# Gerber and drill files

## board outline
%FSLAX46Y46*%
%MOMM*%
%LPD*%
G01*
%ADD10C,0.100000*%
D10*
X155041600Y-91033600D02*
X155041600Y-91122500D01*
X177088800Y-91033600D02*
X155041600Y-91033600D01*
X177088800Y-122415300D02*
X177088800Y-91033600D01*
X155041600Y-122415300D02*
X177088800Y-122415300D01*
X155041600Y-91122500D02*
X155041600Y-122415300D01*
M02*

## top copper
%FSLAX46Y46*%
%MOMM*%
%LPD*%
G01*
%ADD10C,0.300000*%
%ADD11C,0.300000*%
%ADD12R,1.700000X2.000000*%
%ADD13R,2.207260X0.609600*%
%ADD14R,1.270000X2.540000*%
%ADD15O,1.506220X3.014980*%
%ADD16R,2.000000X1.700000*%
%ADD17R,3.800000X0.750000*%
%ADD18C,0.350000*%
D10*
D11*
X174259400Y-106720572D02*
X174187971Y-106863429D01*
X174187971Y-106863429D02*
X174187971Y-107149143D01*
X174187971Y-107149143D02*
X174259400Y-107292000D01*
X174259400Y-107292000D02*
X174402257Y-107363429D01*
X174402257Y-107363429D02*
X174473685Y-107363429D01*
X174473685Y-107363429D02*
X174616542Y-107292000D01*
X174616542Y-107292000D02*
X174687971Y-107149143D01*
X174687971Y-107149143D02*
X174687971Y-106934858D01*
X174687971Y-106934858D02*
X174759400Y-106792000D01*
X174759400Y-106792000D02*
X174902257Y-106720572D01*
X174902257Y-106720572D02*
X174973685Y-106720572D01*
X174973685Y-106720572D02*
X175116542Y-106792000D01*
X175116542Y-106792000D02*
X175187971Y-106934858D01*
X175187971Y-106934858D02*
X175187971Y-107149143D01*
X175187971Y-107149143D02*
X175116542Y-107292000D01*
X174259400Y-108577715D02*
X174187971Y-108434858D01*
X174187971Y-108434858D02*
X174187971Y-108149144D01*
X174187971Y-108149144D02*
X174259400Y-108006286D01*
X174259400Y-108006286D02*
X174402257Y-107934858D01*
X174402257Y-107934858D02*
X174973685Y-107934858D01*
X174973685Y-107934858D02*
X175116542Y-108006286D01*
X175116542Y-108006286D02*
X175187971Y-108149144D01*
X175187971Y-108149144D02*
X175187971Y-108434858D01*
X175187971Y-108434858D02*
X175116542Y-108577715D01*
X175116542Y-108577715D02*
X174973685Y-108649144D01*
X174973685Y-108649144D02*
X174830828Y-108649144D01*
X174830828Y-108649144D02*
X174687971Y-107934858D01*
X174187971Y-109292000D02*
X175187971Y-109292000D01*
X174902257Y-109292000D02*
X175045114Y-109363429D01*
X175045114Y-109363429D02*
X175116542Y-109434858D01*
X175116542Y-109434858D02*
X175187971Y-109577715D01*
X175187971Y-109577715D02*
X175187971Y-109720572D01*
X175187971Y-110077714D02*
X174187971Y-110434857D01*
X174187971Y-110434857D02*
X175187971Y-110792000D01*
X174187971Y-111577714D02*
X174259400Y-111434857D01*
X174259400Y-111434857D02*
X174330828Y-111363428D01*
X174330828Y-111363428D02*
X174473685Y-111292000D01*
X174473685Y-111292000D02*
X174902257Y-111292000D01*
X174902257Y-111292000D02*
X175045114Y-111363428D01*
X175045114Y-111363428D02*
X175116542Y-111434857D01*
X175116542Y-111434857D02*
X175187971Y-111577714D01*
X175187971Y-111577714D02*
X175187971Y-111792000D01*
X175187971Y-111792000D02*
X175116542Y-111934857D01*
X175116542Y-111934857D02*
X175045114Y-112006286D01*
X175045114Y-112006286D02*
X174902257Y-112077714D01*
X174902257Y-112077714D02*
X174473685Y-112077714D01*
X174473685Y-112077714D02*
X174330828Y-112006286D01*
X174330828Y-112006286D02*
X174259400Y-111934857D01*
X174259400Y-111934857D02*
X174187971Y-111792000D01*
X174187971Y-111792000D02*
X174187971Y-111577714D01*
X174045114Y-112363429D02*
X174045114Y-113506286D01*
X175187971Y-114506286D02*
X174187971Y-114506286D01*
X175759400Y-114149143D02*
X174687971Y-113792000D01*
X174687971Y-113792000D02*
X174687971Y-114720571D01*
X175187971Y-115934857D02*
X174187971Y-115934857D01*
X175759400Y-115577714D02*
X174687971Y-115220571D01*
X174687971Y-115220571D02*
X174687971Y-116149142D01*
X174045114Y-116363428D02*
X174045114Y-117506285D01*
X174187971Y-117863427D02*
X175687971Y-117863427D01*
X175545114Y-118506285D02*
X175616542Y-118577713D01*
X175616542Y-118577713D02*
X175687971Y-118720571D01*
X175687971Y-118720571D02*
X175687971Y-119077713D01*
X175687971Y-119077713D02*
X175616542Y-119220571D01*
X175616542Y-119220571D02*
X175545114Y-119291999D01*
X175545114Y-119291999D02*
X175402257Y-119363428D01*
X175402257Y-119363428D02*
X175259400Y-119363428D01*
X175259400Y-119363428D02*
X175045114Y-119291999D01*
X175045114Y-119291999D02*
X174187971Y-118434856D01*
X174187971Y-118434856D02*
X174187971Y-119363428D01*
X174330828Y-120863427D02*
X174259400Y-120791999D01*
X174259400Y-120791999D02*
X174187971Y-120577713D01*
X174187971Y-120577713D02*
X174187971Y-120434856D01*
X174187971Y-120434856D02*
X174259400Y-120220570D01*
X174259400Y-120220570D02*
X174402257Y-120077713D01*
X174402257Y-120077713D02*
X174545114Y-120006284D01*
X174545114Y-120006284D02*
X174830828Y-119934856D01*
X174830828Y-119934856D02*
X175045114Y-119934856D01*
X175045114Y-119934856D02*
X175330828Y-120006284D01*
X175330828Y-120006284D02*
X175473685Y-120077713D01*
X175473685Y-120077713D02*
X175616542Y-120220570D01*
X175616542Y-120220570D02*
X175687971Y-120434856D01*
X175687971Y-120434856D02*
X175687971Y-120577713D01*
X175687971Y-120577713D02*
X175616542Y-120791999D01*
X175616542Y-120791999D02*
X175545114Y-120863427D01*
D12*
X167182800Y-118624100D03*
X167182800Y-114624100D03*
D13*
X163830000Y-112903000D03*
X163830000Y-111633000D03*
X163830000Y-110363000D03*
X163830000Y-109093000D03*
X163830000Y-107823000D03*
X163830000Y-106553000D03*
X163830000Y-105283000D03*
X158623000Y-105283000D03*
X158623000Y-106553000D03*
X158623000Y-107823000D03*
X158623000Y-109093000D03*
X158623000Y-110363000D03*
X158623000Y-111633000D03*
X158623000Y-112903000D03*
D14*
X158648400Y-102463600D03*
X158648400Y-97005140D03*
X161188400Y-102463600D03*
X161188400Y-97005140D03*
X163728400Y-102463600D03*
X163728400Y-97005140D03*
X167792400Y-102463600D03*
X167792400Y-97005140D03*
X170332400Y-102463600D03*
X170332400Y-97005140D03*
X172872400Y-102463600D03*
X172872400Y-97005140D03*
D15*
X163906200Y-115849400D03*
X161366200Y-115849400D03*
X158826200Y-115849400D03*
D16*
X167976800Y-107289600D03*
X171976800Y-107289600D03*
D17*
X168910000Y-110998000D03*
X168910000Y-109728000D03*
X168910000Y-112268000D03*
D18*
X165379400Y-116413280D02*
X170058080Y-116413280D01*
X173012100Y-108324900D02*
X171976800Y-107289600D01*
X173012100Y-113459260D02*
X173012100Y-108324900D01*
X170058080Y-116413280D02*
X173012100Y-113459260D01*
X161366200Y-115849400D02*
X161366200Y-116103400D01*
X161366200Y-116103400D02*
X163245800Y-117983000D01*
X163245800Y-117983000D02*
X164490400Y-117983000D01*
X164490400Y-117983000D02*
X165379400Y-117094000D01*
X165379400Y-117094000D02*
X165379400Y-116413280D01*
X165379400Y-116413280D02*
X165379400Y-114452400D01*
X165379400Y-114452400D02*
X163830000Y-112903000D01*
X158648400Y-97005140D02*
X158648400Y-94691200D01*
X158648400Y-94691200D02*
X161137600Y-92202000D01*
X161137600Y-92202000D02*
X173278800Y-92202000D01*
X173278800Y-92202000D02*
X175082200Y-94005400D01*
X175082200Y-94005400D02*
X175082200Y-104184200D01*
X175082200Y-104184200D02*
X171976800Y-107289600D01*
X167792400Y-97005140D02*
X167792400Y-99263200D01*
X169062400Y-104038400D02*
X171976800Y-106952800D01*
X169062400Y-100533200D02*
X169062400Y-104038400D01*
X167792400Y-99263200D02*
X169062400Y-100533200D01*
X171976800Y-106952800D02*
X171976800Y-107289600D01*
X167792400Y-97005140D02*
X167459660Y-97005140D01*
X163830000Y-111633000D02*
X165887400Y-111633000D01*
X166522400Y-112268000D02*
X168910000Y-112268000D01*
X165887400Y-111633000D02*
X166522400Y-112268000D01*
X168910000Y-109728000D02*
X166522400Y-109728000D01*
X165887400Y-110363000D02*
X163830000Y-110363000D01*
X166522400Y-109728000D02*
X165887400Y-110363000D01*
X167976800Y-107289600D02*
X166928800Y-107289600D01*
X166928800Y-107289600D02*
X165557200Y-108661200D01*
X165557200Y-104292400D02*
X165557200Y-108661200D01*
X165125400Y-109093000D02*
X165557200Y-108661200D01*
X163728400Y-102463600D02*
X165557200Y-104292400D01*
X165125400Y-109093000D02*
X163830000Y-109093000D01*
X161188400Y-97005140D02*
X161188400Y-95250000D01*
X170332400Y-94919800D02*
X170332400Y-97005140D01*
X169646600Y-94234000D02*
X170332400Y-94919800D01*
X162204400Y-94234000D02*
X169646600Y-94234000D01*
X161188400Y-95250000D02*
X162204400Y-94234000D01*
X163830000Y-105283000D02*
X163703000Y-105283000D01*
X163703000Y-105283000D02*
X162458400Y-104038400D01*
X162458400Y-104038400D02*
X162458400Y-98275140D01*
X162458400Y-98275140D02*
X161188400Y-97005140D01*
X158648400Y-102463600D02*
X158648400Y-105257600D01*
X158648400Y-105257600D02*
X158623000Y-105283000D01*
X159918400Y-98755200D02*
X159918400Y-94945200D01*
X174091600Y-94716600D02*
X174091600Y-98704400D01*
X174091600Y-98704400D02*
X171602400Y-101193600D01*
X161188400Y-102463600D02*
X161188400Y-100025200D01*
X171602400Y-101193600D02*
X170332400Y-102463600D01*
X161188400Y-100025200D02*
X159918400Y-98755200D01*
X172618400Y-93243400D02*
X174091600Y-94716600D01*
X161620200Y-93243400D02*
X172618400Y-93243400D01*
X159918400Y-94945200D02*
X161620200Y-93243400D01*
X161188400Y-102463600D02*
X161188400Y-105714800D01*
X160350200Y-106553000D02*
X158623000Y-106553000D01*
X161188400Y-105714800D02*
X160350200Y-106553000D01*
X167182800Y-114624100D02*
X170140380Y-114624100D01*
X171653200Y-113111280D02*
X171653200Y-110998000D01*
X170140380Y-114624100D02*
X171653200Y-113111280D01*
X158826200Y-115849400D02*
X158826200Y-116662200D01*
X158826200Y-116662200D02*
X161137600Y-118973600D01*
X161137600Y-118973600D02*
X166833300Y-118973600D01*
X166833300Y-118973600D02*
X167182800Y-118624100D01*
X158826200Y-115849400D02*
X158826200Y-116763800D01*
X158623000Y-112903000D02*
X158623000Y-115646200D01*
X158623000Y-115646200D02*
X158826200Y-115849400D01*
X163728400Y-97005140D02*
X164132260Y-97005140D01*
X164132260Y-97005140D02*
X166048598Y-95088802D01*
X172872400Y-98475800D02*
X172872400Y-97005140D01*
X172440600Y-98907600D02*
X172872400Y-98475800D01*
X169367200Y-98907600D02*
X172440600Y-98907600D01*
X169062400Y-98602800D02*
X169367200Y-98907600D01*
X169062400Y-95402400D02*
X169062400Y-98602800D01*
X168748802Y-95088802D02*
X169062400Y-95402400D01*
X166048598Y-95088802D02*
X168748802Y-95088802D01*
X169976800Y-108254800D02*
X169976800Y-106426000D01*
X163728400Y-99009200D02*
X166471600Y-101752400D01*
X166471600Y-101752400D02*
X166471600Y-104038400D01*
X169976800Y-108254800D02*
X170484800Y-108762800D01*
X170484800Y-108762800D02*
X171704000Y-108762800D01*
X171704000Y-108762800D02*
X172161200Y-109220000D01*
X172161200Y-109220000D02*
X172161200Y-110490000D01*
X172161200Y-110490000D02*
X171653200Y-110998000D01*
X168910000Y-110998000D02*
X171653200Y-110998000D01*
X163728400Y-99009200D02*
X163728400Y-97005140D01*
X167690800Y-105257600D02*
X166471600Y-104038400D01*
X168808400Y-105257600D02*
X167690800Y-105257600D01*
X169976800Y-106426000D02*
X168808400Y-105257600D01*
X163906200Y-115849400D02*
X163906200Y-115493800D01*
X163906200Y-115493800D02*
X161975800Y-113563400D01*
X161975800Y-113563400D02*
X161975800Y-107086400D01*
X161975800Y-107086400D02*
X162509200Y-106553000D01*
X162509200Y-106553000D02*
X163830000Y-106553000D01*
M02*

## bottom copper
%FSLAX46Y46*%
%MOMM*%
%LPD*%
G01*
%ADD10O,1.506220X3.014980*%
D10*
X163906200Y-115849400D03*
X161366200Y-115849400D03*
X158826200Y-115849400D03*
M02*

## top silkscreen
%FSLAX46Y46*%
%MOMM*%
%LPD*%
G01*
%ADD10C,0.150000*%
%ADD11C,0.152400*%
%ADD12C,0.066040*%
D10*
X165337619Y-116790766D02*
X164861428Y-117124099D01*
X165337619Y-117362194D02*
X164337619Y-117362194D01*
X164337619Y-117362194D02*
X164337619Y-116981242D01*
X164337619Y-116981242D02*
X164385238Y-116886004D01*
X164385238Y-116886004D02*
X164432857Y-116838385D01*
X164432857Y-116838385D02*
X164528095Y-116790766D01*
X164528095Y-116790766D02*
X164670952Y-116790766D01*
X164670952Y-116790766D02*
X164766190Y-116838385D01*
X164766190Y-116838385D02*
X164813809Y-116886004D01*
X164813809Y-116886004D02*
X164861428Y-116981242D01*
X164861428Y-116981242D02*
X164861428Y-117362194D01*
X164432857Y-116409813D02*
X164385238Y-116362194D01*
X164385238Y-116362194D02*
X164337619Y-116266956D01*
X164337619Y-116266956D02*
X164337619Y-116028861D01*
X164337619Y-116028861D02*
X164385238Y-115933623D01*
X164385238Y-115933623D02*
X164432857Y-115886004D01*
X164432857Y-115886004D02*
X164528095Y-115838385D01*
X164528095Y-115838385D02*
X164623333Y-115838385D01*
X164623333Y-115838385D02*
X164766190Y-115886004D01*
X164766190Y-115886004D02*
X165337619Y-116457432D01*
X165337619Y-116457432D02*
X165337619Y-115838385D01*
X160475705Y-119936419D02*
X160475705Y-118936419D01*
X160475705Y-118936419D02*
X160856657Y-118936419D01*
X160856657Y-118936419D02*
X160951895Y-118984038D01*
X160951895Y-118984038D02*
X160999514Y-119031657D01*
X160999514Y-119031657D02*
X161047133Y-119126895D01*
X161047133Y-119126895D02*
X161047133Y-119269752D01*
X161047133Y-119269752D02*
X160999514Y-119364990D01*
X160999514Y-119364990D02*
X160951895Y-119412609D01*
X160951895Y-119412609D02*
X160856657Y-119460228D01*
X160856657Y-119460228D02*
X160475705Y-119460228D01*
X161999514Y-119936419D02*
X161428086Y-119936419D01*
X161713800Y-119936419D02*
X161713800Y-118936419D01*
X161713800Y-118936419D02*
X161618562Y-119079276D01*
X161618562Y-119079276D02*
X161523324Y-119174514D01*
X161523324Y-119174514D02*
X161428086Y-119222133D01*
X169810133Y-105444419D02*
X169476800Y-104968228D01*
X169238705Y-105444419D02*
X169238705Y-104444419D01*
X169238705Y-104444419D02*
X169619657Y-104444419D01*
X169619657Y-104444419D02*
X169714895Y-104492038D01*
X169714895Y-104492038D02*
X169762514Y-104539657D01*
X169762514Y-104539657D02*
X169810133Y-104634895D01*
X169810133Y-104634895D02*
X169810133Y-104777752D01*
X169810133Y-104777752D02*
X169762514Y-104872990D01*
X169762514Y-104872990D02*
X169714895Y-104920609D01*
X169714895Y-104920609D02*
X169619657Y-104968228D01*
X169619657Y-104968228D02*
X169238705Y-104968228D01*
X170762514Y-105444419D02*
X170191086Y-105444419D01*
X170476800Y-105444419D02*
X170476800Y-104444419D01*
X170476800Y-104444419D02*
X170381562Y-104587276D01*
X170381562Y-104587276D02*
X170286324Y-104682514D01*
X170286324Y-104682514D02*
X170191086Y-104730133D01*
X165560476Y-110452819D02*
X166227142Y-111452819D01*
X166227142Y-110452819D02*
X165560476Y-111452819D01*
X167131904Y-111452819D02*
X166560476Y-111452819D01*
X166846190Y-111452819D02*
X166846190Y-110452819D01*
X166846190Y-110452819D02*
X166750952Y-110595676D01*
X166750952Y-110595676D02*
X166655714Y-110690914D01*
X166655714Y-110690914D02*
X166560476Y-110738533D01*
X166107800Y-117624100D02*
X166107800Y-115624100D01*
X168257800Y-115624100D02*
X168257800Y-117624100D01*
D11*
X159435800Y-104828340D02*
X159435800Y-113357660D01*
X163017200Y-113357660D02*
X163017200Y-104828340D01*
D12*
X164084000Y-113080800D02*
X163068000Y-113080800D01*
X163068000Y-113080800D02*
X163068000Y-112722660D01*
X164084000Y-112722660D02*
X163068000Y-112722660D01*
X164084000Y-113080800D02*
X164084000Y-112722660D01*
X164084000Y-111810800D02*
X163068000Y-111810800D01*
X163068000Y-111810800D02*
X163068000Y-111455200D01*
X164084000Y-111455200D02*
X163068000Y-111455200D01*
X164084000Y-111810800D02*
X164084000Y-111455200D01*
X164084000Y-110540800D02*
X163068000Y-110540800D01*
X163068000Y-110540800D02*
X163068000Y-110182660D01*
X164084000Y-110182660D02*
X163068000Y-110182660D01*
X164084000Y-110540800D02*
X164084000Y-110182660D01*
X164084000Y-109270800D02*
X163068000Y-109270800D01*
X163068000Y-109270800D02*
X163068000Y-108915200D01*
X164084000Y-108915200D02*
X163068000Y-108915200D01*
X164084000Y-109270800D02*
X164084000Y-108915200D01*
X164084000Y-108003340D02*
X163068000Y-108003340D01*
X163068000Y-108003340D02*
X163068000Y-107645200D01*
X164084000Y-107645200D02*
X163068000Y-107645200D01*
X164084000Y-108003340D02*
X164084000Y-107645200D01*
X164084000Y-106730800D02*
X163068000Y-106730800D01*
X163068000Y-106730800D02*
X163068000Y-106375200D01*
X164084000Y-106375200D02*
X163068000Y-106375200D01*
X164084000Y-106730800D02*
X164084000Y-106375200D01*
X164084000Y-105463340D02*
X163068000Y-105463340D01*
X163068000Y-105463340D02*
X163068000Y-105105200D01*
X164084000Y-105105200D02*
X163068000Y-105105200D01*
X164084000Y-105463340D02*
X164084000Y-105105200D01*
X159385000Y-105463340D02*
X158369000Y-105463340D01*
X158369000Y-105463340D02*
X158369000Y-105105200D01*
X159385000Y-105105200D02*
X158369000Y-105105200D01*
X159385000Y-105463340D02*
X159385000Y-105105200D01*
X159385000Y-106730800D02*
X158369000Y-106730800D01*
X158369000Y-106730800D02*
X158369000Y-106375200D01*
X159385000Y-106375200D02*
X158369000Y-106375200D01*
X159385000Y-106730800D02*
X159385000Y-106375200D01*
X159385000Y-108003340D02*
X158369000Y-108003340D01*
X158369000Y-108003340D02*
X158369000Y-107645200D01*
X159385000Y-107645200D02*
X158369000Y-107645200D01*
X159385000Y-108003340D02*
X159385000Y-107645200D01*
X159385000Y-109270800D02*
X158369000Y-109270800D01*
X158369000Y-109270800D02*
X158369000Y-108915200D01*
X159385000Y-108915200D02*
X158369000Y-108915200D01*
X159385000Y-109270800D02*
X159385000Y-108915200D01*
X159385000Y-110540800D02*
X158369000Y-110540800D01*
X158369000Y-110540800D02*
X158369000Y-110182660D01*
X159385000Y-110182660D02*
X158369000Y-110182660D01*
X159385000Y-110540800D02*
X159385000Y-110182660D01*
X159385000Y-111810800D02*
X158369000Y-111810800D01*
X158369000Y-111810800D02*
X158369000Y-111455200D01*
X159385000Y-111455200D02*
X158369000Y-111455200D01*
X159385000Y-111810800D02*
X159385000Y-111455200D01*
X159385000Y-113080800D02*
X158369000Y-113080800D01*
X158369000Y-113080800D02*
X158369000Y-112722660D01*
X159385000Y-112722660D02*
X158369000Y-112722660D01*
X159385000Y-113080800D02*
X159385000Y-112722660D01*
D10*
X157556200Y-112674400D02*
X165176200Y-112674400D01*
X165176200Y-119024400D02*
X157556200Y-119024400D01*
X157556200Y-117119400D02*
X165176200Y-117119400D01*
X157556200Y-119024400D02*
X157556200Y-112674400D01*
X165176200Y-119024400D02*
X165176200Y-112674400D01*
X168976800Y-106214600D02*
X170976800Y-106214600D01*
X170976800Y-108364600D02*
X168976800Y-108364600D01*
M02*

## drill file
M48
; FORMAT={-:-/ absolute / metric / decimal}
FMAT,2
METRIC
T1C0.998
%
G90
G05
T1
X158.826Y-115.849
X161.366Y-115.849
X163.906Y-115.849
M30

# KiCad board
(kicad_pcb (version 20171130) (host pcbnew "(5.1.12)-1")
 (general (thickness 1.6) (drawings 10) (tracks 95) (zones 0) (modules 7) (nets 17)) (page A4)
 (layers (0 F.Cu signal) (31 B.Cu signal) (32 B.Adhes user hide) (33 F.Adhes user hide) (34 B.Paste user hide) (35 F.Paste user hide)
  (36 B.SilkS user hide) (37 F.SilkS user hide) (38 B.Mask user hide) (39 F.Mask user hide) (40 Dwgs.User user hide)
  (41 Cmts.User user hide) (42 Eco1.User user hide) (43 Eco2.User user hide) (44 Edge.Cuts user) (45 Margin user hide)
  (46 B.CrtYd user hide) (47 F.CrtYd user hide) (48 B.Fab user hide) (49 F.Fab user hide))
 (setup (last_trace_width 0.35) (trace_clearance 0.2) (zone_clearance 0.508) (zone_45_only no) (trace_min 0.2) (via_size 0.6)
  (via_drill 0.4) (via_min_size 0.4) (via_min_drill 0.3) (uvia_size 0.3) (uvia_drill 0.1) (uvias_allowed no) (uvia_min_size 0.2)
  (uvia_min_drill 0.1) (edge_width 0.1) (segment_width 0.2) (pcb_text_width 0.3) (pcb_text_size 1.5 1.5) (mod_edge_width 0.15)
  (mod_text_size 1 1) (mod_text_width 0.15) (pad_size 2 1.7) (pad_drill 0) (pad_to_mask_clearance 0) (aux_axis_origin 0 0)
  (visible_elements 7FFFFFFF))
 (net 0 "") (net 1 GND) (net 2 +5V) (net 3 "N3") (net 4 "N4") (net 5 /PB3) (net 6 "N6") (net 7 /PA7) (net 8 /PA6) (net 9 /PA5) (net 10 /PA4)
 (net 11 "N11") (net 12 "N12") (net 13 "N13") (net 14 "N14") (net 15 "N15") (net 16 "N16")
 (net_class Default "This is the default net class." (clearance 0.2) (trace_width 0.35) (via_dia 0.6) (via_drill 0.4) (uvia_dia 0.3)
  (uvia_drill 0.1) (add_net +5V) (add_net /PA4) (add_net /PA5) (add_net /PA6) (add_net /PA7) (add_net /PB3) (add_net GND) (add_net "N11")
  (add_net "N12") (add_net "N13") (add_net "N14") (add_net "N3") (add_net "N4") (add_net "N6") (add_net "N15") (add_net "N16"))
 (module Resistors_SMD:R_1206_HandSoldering (layer F.Cu) (at 167.1828 116.6241 90)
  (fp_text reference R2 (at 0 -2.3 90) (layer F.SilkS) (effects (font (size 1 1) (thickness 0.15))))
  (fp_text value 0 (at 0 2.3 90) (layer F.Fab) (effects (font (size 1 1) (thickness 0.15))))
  (fp_line (start -1 -1.075) (end 1 -1.075) (layer F.SilkS) (width 0.15))
  (fp_line (start 1 1.075) (end -1 1.075) (layer F.SilkS) (width 0.15))
  (pad 2 smd rect (at -2 0 90) (size 2 1.7) (layers F.Cu F.Paste F.Mask) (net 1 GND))
  (pad 1 smd rect (at 2 0 90) (size 2 1.7) (layers F.Cu F.Paste F.Mask) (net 1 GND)))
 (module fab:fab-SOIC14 (layer F.Cu) (at 161.2265 109.093 90)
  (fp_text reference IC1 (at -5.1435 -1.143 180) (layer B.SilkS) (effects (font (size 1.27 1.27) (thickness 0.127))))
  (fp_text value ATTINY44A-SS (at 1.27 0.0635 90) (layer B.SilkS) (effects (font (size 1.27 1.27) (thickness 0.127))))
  (fp_line (start 4.26466 -1.7907) (end -4.26466 -1.7907) (layer F.SilkS) (width 0.1524))
  (fp_line (start -4.26466 1.7907) (end 4.26466 1.7907) (layer F.SilkS) (width 0.1524))
  (fp_line (start -3.9878 2.8575) (end -3.9878 1.8415) (layer F.SilkS) (width 0.06604))
  (fp_line (start -3.9878 1.8415) (end -3.62966 1.8415) (layer F.SilkS) (width 0.06604))
  (fp_line (start -3.62966 2.8575) (end -3.62966 1.8415) (layer F.SilkS) (width 0.06604))
  (fp_line (start -3.9878 2.8575) (end -3.62966 2.8575) (layer F.SilkS) (width 0.06604))
  (fp_line (start -2.7178 2.8575) (end -2.7178 1.8415) (layer F.SilkS) (width 0.06604))
  (fp_line (start -2.7178 1.8415) (end -2.3622 1.8415) (layer F.SilkS) (width 0.06604))
  (fp_line (start -2.3622 2.8575) (end -2.3622 1.8415) (layer F.SilkS) (width 0.06604))
  (fp_line (start -2.7178 2.8575) (end -2.3622 2.8575) (layer F.SilkS) (width 0.06604))
  (fp_line (start -1.4478 2.8575) (end -1.4478 1.8415) (layer F.SilkS) (width 0.06604))
  (fp_line (start -1.4478 1.8415) (end -1.08966 1.8415) (layer F.SilkS) (width 0.06604))
  (fp_line (start -1.08966 2.8575) (end -1.08966 1.8415) (layer F.SilkS) (width 0.06604))
  (fp_line (start -1.4478 2.8575) (end -1.08966 2.8575) (layer F.SilkS) (width 0.06604))
  (fp_line (start -0.1778 2.8575) (end -0.1778 1.8415) (layer F.SilkS) (width 0.06604))
  (fp_line (start -0.1778 1.8415) (end 0.1778 1.8415) (layer F.SilkS) (width 0.06604))
  (fp_line (start 0.1778 2.8575) (end 0.1778 1.8415) (layer F.SilkS) (width 0.06604))
  (fp_line (start -0.1778 2.8575) (end 0.1778 2.8575) (layer F.SilkS) (width 0.06604))
  (fp_line (start 1.08966 2.8575) (end 1.08966 1.8415) (layer F.SilkS) (width 0.06604))
  (fp_line (start 1.08966 1.8415) (end 1.4478 1.8415) (layer F.SilkS) (width 0.06604))
  (fp_line (start 1.4478 2.8575) (end 1.4478 1.8415) (layer F.SilkS) (width 0.06604))
  (fp_line (start 1.08966 2.8575) (end 1.4478 2.8575) (layer F.SilkS) (width 0.06604))
  (fp_line (start 2.3622 2.8575) (end 2.3622 1.8415) (layer F.SilkS) (width 0.06604))
  (fp_line (start 2.3622 1.8415) (end 2.7178 1.8415) (layer F.SilkS) (width 0.06604))
  (fp_line (start 2.7178 2.8575) (end 2.7178 1.8415) (layer F.SilkS) (width 0.06604))
  (fp_line (start 2.3622 2.8575) (end 2.7178 2.8575) (layer F.SilkS) (width 0.06604))
  (fp_line (start 3.62966 2.8575) (end 3.62966 1.8415) (layer F.SilkS) (width 0.06604))
  (fp_line (start 3.62966 1.8415) (end 3.9878 1.8415) (layer F.SilkS) (width 0.06604))
  (fp_line (start 3.9878 2.8575) (end 3.9878 1.8415) (layer F.SilkS) (width 0.06604))
  (fp_line (start 3.62966 2.8575) (end 3.9878 2.8575) (layer F.SilkS) (width 0.06604))
  (fp_line (start 3.62966 -1.8415) (end 3.62966 -2.8575) (layer F.SilkS) (width 0.06604))
  (fp_line (start 3.62966 -2.8575) (end 3.9878 -2.8575) (layer F.SilkS) (width 0.06604))
  (fp_line (start 3.9878 -1.8415) (end 3.9878 -2.8575) (layer F.SilkS) (width 0.06604))
  (fp_line (start 3.62966 -1.8415) (end 3.9878 -1.8415) (layer F.SilkS) (width 0.06604))
  (fp_line (start 2.3622 -1.8415) (end 2.3622 -2.8575) (layer F.SilkS) (width 0.06604))
  (fp_line (start 2.3622 -2.8575) (end 2.7178 -2.8575) (layer F.SilkS) (width 0.06604))
  (fp_line (start 2.7178 -1.8415) (end 2.7178 -2.8575) (layer F.SilkS) (width 0.06604))
  (fp_line (start 2.3622 -1.8415) (end 2.7178 -1.8415) (layer F.SilkS) (width 0.06604))
  (fp_line (start 1.08966 -1.8415) (end 1.08966 -2.8575) (layer F.SilkS) (width 0.06604))
  (fp_line (start 1.08966 -2.8575) (end 1.4478 -2.8575) (layer F.SilkS) (width 0.06604))
  (fp_line (start 1.4478 -1.8415) (end 1.4478 -2.8575) (layer F.SilkS) (width 0.06604))
  (fp_line (start 1.08966 -1.8415) (end 1.4478 -1.8415) (layer F.SilkS) (width 0.06604))
  (fp_line (start -0.1778 -1.8415) (end -0.1778 -2.8575) (layer F.SilkS) (width 0.06604))
  (fp_line (start -0.1778 -2.8575) (end 0.1778 -2.8575) (layer F.SilkS) (width 0.06604))
  (fp_line (start 0.1778 -1.8415) (end 0.1778 -2.8575) (layer F.SilkS) (width 0.06604))
  (fp_line (start -0.1778 -1.8415) (end 0.1778 -1.8415) (layer F.SilkS) (width 0.06604))
  (fp_line (start -1.4478 -1.8415) (end -1.4478 -2.8575) (layer F.SilkS) (width 0.06604))
  (fp_line (start -1.4478 -2.8575) (end -1.08966 -2.8575) (layer F.SilkS) (width 0.06604))
  (fp_line (start -1.08966 -1.8415) (end -1.08966 -2.8575) (layer F.SilkS) (width 0.06604))
  (fp_line (start -1.4478 -1.8415) (end -1.08966 -1.8415) (layer F.SilkS) (width 0.06604))
  (fp_line (start -2.7178 -1.8415) (end -2.7178 -2.8575) (layer F.SilkS) (width 0.06604))
  (fp_line (start -2.7178 -2.8575) (end -2.3622 -2.8575) (layer F.SilkS) (width 0.06604))
  (fp_line (start -2.3622 -1.8415) (end -2.3622 -2.8575) (layer F.SilkS) (width 0.06604))
  (fp_line (start -2.7178 -1.8415) (end -2.3622 -1.8415) (layer F.SilkS) (width 0.06604))
  (fp_line (start -3.9878 -1.8415) (end -3.9878 -2.8575) (layer F.SilkS) (width 0.06604))
  (fp_line (start -3.9878 -2.8575) (end -3.62966 -2.8575) (layer F.SilkS) (width 0.06604))
  (fp_line (start -3.62966 -1.8415) (end -3.62966 -2.8575) (layer F.SilkS) (width 0.06604))
  (fp_line (start -3.9878 -1.8415) (end -3.62966 -1.8415) (layer F.SilkS) (width 0.06604))
  (pad 1 smd rect (at -3.81 2.6035 90) (size 0.6096 2.20726) (layers F.Cu F.Paste F.Mask) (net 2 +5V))
  (pad 2 smd rect (at -2.54 2.6035 90) (size 0.6096 2.20726) (layers F.Cu F.Paste F.Mask) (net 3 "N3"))
  (pad 3 smd rect (at -1.27 2.6035 90) (size 0.6096 2.20726) (layers F.Cu F.Paste F.Mask) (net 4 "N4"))
  (pad 4 smd rect (at 0 2.6035 90) (size 0.6096 2.20726) (layers F.Cu F.Paste F.Mask) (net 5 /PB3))
  (pad 5 smd rect (at 1.27 2.6035 90) (size 0.6096 2.20726) (layers F.Cu F.Paste F.Mask) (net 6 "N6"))
  (pad 6 smd rect (at 2.54 2.6035 90) (size 0.6096 2.20726) (layers F.Cu F.Paste F.Mask) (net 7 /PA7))
  (pad 7 smd rect (at 3.81 2.6035 90) (size 0.6096 2.20726) (layers F.Cu F.Paste F.Mask) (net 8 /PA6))
  (pad 8 smd rect (at 3.81 -2.6035 90) (size 0.6096 2.20726) (layers F.Cu F.Paste F.Mask) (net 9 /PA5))
  (pad 9 smd rect (at 2.54 -2.6035 90) (size 0.6096 2.20726) (layers F.Cu F.Paste F.Mask) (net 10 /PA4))
  (pad 10 smd rect (at 1.27 -2.6035 90) (size 0.6096 2.20726) (layers F.Cu F.Paste F.Mask) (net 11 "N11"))
  (pad 11 smd rect (at 0 -2.6035 90) (size 0.6096 2.20726) (layers F.Cu F.Paste F.Mask) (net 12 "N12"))
  (pad 12 smd rect (at -1.27 -2.6035 90) (size 0.6096 2.20726) (layers F.Cu F.Paste F.Mask) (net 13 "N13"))
  (pad 13 smd rect (at -2.54 -2.6035 90) (size 0.6096 2.20726) (layers F.Cu F.Paste F.Mask) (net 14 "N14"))
  (pad 14 smd rect (at -3.81 -2.6035 90) (size 0.6096 2.20726) (layers F.Cu F.Paste F.Mask) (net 1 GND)))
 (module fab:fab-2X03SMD (layer F.Cu) (at 161.1884 99.9236 90)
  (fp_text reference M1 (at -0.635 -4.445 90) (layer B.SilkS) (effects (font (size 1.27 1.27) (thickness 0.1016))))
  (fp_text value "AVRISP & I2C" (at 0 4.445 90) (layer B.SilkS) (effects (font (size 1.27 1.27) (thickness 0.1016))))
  (pad 1 smd rect (at -2.54 -2.54 90) (size 2.54 1.27) (layers F.Cu F.Paste F.Mask) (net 9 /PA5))
  (pad 2 smd rect (at 2.91846 -2.54 90) (size 2.54 1.27) (layers F.Cu F.Paste F.Mask) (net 2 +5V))
  (pad 3 smd rect (at -2.54 0 90) (size 2.54 1.27) (layers F.Cu F.Paste F.Mask) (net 10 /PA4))
  (pad 4 smd rect (at 2.91846 0 90) (size 2.54 1.27) (layers F.Cu F.Paste F.Mask) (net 8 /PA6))
  (pad 5 smd rect (at -2.54 2.54 90) (size 2.54 1.27) (layers F.Cu F.Paste F.Mask) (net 5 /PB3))
  (pad 6 smd rect (at 2.91846 2.54 90) (size 2.54 1.27) (layers F.Cu F.Paste F.Mask) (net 1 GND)))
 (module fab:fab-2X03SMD (layer F.Cu) (at 170.3324 99.9236 90)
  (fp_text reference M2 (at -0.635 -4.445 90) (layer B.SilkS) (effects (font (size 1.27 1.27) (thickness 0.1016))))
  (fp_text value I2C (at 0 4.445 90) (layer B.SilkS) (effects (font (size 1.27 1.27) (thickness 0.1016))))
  (pad 1 smd rect (at -2.54 -2.54 90) (size 2.54 1.27) (layers F.Cu F.Paste F.Mask) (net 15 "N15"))
  (pad 2 smd rect (at 2.91846 -2.54 90) (size 2.54 1.27) (layers F.Cu F.Paste F.Mask) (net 2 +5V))
  (pad 3 smd rect (at -2.54 0 90) (size 2.54 1.27) (layers F.Cu F.Paste F.Mask) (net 10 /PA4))
  (pad 4 smd rect (at 2.91846 0 90) (size 2.54 1.27) (layers F.Cu F.Paste F.Mask) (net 8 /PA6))
  (pad 5 smd rect (at -2.54 2.54 90) (size 2.54 1.27) (layers F.Cu F.Paste F.Mask) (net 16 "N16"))
  (pad 6 smd rect (at 2.91846 2.54 90) (size 2.54 1.27) (layers F.Cu F.Paste F.Mask) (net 1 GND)))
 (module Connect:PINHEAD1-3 (layer F.Cu) (at 161.3662 115.8494 180)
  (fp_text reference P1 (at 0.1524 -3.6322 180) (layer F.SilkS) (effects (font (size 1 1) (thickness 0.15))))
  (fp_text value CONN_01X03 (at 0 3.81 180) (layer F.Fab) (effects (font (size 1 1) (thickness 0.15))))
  (fp_line (start 3.81 3.175) (end -3.81 3.175) (layer F.SilkS) (width 0.15))
  (fp_line (start -3.81 -3.175) (end 3.81 -3.175) (layer F.SilkS) (width 0.15))
  (fp_line (start 3.81 -1.27) (end -3.81 -1.27) (layer F.SilkS) (width 0.15))
  (fp_line (start 3.81 -3.175) (end 3.81 3.175) (layer F.SilkS) (width 0.15))
  (fp_line (start -3.81 -3.175) (end -3.81 3.175) (layer F.SilkS) (width 0.15))
  (pad 1 thru_hole oval (at -2.54 0 180) (size 1.50622 3.01498) (drill 0.99822) (layers *.Cu *.Mask) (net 7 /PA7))
  (pad 2 thru_hole oval (at 0 0 180) (size 1.50622 3.01498) (drill 0.99822) (layers *.Cu *.Mask) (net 2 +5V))
  (pad 3 thru_hole oval (at 2.54 0 180) (size 1.50622 3.01498) (drill 0.99822) (layers *.Cu *.Mask) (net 1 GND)))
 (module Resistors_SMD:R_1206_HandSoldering (layer F.Cu) (at 169.9768 107.2896)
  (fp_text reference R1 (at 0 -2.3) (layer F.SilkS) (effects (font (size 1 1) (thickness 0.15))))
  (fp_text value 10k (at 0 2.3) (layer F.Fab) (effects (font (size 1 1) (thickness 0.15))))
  (fp_line (start -1 -1.075) (end 1 -1.075) (layer F.SilkS) (width 0.15))
  (fp_line (start 1 1.075) (end -1 1.075) (layer F.SilkS) (width 0.15))
  (pad 1 smd rect (at -2 0) (size 2 1.7) (layers F.Cu F.Paste F.Mask) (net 5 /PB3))
  (pad 2 smd rect (at 2 0) (size 2 1.7) (layers F.Cu F.Paste F.Mask) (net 2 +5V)))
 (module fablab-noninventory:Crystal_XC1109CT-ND (layer F.Cu) (at 168.91 110.998 90)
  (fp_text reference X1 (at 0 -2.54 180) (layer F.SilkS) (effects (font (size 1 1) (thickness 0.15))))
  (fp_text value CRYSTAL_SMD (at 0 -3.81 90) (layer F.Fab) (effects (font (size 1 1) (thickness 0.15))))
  (pad 2 smd rect (at 0 0 90) (size 0.75 3.8) (layers F.Cu F.Paste F.Mask) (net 1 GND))
  (pad 1 smd rect (at 1.27 0 90) (size 0.75 3.8) (layers F.Cu F.Paste F.Mask) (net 4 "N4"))
  (pad 3 smd rect (at -1.27 0 90) (size 0.75 3.8) (layers F.Cu F.Paste F.Mask) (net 3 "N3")))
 (gr_line (start 155.0416 91.0336) (end 155.0416 91.1225) (angle 90) (layer Edge.Cuts) (width 0.1))
 (gr_line (start 177.0888 91.0336) (end 155.0416 91.0336) (angle 90) (layer Edge.Cuts) (width 0.1))
 (gr_line (start 177.0888 122.4153) (end 177.0888 91.0336) (angle 90) (layer Edge.Cuts) (width 0.1))
 (gr_line (start 155.0416 122.4153) (end 177.0888 122.4153) (angle 90) (layer Edge.Cuts) (width 0.1))
 (gr_line (start 155.0416 91.1225) (end 155.0416 122.4153) (angle 90) (layer Edge.Cuts) (width 0.1))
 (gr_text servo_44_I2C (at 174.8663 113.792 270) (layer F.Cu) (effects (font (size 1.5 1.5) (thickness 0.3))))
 (segment (start 165.3794 116.41328) (end 170.05808 116.41328) (width 0.35) (layer F.Cu) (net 2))
 (segment (start 173.0121 108.3249) (end 171.9768 107.2896) (width 0.35) (layer F.Cu) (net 2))
 (segment (start 173.0121 113.45926) (end 173.0121 108.3249) (width 0.35) (layer F.Cu) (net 2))
 (segment (start 170.05808 116.41328) (end 173.0121 113.45926) (width 0.35) (layer F.Cu) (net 2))
 (segment (start 161.3662 115.8494) (end 161.3662 116.1034) (width 0.35) (layer F.Cu) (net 2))
 (segment (start 161.3662 116.1034) (end 163.2458 117.983) (width 0.35) (layer F.Cu) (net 2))
 (segment (start 163.2458 117.983) (end 164.4904 117.983) (width 0.35) (layer F.Cu) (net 2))
 (segment (start 164.4904 117.983) (end 165.3794 117.094) (width 0.35) (layer F.Cu) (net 2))
 (segment (start 165.3794 117.094) (end 165.3794 116.41328) (width 0.35) (layer F.Cu) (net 2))
 (segment (start 165.3794 116.41328) (end 165.3794 114.4524) (width 0.35) (layer F.Cu) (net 2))
 (segment (start 165.3794 114.4524) (end 163.83 112.903) (width 0.35) (layer F.Cu) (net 2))
 (segment (start 158.6484 97.00514) (end 158.6484 94.6912) (width 0.35) (layer F.Cu) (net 2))
 (segment (start 158.6484 94.6912) (end 161.1376 92.202) (width 0.35) (layer F.Cu) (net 2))
 (segment (start 161.1376 92.202) (end 173.2788 92.202) (width 0.35) (layer F.Cu) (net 2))
 (segment (start 173.2788 92.202) (end 175.0822 94.0054) (width 0.35) (layer F.Cu) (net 2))
 (segment (start 175.0822 94.0054) (end 175.0822 104.1842) (width 0.35) (layer F.Cu) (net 2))
 (segment (start 175.0822 104.1842) (end 171.9768 107.2896) (width 0.35) (layer F.Cu) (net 2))
 (segment (start 167.7924 97.00514) (end 167.7924 99.2632) (width 0.35) (layer F.Cu) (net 2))
 (segment (start 169.0624 104.0384) (end 171.9768 106.9528) (width 0.35) (layer F.Cu) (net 2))
 (segment (start 169.0624 100.5332) (end 169.0624 104.0384) (width 0.35) (layer F.Cu) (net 2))
 (segment (start 167.7924 99.2632) (end 169.0624 100.5332) (width 0.35) (layer F.Cu) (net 2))
 (segment (start 171.9768 106.9528) (end 171.9768 107.2896) (width 0.35) (layer F.Cu) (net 2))
 (segment (start 167.7924 97.00514) (end 167.45966 97.00514) (width 0.35) (layer F.Cu) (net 2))
 (segment (start 163.83 111.633) (end 165.8874 111.633) (width 0.35) (layer F.Cu) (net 3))
 (segment (start 166.5224 112.268) (end 168.91 112.268) (width 0.35) (layer F.Cu) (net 3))
 (segment (start 165.8874 111.633) (end 166.5224 112.268) (width 0.35) (layer F.Cu) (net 3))
 (segment (start 168.91 109.728) (end 166.5224 109.728) (width 0.35) (layer F.Cu) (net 4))
 (segment (start 165.8874 110.363) (end 163.83 110.363) (width 0.35) (layer F.Cu) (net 4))
 (segment (start 166.5224 109.728) (end 165.8874 110.363) (width 0.35) (layer F.Cu) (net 4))
 (segment (start 167.9768 107.2896) (end 166.9288 107.2896) (width 0.35) (layer F.Cu) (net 5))
 (segment (start 166.9288 107.2896) (end 165.5572 108.6612) (width 0.35) (layer F.Cu) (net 5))
 (segment (start 165.5572 104.2924) (end 165.5572 108.6612) (width 0.35) (layer F.Cu) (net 5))
 (segment (start 165.1254 109.093) (end 165.5572 108.6612) (width 0.35) (layer F.Cu) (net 5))
 (segment (start 163.7284 102.4636) (end 165.5572 104.2924) (width 0.35) (layer F.Cu) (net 5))
 (segment (start 165.1254 109.093) (end 163.83 109.093) (width 0.35) (layer F.Cu) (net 5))
 (segment (start 161.1884 97.00514) (end 161.1884 95.25) (width 0.35) (layer F.Cu) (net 8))
 (segment (start 170.3324 94.9198) (end 170.3324 97.00514) (width 0.35) (layer F.Cu) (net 8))
 (segment (start 169.6466 94.234) (end 170.3324 94.9198) (width 0.35) (layer F.Cu) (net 8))
 (segment (start 162.2044 94.234) (end 169.6466 94.234) (width 0.35) (layer F.Cu) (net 8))
 (segment (start 161.1884 95.25) (end 162.2044 94.234) (width 0.35) (layer F.Cu) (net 8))
 (segment (start 163.83 105.283) (end 163.703 105.283) (width 0.35) (layer F.Cu) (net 8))
 (segment (start 163.703 105.283) (end 162.4584 104.0384) (width 0.35) (layer F.Cu) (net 8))
 (segment (start 162.4584 104.0384) (end 162.4584 98.27514) (width 0.35) (layer F.Cu) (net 8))
 (segment (start 162.4584 98.27514) (end 161.1884 97.00514) (width 0.35) (layer F.Cu) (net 8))
 (segment (start 158.6484 102.4636) (end 158.6484 105.2576) (width 0.35) (layer F.Cu) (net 9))
 (segment (start 158.6484 105.2576) (end 158.623 105.283) (width 0.35) (layer F.Cu) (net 9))
 (segment (start 159.9184 98.7552) (end 159.9184 94.9452) (width 0.35) (layer F.Cu) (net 10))
 (segment (start 174.0916 94.7166) (end 174.0916 98.7044) (width 0.35) (layer F.Cu) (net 10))
 (segment (start 174.0916 98.7044) (end 171.6024 101.1936) (width 0.35) (layer F.Cu) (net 10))
 (segment (start 161.1884 102.4636) (end 161.1884 100.0252) (width 0.35) (layer F.Cu) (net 10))
 (segment (start 171.6024 101.1936) (end 170.3324 102.4636) (width 0.35) (layer F.Cu) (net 10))
 (segment (start 161.1884 100.0252) (end 159.9184 98.7552) (width 0.35) (layer F.Cu) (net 10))
 (segment (start 172.6184 93.2434) (end 174.0916 94.7166) (width 0.35) (layer F.Cu) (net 10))
 (segment (start 161.6202 93.2434) (end 172.6184 93.2434) (width 0.35) (layer F.Cu) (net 10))
 (segment (start 159.9184 94.9452) (end 161.6202 93.2434) (width 0.35) (layer F.Cu) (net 10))
 (segment (start 161.1884 102.4636) (end 161.1884 105.7148) (width 0.35) (layer F.Cu) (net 10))
 (segment (start 160.3502 106.553) (end 158.623 106.553) (width 0.35) (layer F.Cu) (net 10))
 (segment (start 161.1884 105.7148) (end 160.3502 106.553) (width 0.35) (layer F.Cu) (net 10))
 (segment (start 167.1828 114.6241) (end 170.14038 114.6241) (width 0.35) (layer F.Cu) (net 1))
 (segment (start 171.6532 113.11128) (end 171.6532 110.998) (width 0.35) (layer F.Cu) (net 1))
 (segment (start 170.14038 114.6241) (end 171.6532 113.11128) (width 0.35) (layer F.Cu) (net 1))
 (segment (start 158.8262 115.8494) (end 158.8262 116.6622) (width 0.35) (layer F.Cu) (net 1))
 (segment (start 158.8262 116.6622) (end 161.1376 118.9736) (width 0.35) (layer F.Cu) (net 1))
 (segment (start 161.1376 118.9736) (end 166.8333 118.9736) (width 0.35) (layer F.Cu) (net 1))
 (segment (start 166.8333 118.9736) (end 167.1828 118.6241) (width 0.35) (layer F.Cu) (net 1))
 (segment (start 158.8262 115.8494) (end 158.8262 116.7638) (width 0.35) (layer F.Cu) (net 1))
 (segment (start 158.623 112.903) (end 158.623 115.6462) (width 0.35) (layer F.Cu) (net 1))
 (segment (start 158.623 115.6462) (end 158.8262 115.8494) (width 0.35) (layer F.Cu) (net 1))
 (segment (start 163.7284 97.00514) (end 164.13226 97.00514) (width 0.35) (layer F.Cu) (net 1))
 (segment (start 164.13226 97.00514) (end 166.048598 95.088802) (width 0.35) (layer F.Cu) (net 1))
 (segment (start 172.8724 98.4758) (end 172.8724 97.00514) (width 0.35) (layer F.Cu) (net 1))
 (segment (start 172.4406 98.9076) (end 172.8724 98.4758) (width 0.35) (layer F.Cu) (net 1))
 (segment (start 169.3672 98.9076) (end 172.4406 98.9076) (width 0.35) (layer F.Cu) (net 1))
 (segment (start 169.0624 98.6028) (end 169.3672 98.9076) (width 0.35) (layer F.Cu) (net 1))
 (segment (start 169.0624 95.4024) (end 169.0624 98.6028) (width 0.35) (layer F.Cu) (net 1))
 (segment (start 168.748802 95.088802) (end 169.0624 95.4024) (width 0.35) (layer F.Cu) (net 1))
 (segment (start 166.048598 95.088802) (end 168.748802 95.088802) (width 0.35) (layer F.Cu) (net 1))
 (segment (start 169.9768 108.2548) (end 169.9768 106.426) (width 0.35) (layer F.Cu) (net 1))
 (segment (start 163.7284 99.0092) (end 166.4716 101.7524) (width 0.35) (layer F.Cu) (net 1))
 (segment (start 166.4716 101.7524) (end 166.4716 104.0384) (width 0.35) (layer F.Cu) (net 1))
 (segment (start 169.9768 108.2548) (end 170.4848 108.7628) (width 0.35) (layer F.Cu) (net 1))
 (segment (start 170.4848 108.7628) (end 171.704 108.7628) (width 0.35) (layer F.Cu) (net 1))
 (segment (start 171.704 108.7628) (end 172.1612 109.22) (width 0.35) (layer F.Cu) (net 1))
 (segment (start 172.1612 109.22) (end 172.1612 110.49) (width 0.35) (layer F.Cu) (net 1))
 (segment (start 172.1612 110.49) (end 171.6532 110.998) (width 0.35) (layer F.Cu) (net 1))
 (segment (start 168.91 110.998) (end 171.6532 110.998) (width 0.35) (layer F.Cu) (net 1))
 (segment (start 163.7284 99.0092) (end 163.7284 97.00514) (width 0.35) (layer F.Cu) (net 1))
 (segment (start 167.6908 105.2576) (end 166.4716 104.0384) (width 0.35) (layer F.Cu) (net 1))
 (segment (start 168.8084 105.2576) (end 167.6908 105.2576) (width 0.35) (layer F.Cu) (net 1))
 (segment (start 169.9768 106.426) (end 168.8084 105.2576) (width 0.35) (layer F.Cu) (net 1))
 (segment (start 163.9062 115.8494) (end 163.9062 115.4938) (width 0.35) (layer F.Cu) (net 7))
 (segment (start 163.9062 115.4938) (end 161.9758 113.5634) (width 0.35) (layer F.Cu) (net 7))
 (segment (start 161.9758 113.5634) (end 161.9758 107.0864) (width 0.35) (layer F.Cu) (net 7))
 (segment (start 161.9758 107.0864) (end 162.5092 106.553) (width 0.35) (layer F.Cu) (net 7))
 (segment (start 162.5092 106.553) (end 163.83 106.553) (width 0.35) (layer F.Cu) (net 7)))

